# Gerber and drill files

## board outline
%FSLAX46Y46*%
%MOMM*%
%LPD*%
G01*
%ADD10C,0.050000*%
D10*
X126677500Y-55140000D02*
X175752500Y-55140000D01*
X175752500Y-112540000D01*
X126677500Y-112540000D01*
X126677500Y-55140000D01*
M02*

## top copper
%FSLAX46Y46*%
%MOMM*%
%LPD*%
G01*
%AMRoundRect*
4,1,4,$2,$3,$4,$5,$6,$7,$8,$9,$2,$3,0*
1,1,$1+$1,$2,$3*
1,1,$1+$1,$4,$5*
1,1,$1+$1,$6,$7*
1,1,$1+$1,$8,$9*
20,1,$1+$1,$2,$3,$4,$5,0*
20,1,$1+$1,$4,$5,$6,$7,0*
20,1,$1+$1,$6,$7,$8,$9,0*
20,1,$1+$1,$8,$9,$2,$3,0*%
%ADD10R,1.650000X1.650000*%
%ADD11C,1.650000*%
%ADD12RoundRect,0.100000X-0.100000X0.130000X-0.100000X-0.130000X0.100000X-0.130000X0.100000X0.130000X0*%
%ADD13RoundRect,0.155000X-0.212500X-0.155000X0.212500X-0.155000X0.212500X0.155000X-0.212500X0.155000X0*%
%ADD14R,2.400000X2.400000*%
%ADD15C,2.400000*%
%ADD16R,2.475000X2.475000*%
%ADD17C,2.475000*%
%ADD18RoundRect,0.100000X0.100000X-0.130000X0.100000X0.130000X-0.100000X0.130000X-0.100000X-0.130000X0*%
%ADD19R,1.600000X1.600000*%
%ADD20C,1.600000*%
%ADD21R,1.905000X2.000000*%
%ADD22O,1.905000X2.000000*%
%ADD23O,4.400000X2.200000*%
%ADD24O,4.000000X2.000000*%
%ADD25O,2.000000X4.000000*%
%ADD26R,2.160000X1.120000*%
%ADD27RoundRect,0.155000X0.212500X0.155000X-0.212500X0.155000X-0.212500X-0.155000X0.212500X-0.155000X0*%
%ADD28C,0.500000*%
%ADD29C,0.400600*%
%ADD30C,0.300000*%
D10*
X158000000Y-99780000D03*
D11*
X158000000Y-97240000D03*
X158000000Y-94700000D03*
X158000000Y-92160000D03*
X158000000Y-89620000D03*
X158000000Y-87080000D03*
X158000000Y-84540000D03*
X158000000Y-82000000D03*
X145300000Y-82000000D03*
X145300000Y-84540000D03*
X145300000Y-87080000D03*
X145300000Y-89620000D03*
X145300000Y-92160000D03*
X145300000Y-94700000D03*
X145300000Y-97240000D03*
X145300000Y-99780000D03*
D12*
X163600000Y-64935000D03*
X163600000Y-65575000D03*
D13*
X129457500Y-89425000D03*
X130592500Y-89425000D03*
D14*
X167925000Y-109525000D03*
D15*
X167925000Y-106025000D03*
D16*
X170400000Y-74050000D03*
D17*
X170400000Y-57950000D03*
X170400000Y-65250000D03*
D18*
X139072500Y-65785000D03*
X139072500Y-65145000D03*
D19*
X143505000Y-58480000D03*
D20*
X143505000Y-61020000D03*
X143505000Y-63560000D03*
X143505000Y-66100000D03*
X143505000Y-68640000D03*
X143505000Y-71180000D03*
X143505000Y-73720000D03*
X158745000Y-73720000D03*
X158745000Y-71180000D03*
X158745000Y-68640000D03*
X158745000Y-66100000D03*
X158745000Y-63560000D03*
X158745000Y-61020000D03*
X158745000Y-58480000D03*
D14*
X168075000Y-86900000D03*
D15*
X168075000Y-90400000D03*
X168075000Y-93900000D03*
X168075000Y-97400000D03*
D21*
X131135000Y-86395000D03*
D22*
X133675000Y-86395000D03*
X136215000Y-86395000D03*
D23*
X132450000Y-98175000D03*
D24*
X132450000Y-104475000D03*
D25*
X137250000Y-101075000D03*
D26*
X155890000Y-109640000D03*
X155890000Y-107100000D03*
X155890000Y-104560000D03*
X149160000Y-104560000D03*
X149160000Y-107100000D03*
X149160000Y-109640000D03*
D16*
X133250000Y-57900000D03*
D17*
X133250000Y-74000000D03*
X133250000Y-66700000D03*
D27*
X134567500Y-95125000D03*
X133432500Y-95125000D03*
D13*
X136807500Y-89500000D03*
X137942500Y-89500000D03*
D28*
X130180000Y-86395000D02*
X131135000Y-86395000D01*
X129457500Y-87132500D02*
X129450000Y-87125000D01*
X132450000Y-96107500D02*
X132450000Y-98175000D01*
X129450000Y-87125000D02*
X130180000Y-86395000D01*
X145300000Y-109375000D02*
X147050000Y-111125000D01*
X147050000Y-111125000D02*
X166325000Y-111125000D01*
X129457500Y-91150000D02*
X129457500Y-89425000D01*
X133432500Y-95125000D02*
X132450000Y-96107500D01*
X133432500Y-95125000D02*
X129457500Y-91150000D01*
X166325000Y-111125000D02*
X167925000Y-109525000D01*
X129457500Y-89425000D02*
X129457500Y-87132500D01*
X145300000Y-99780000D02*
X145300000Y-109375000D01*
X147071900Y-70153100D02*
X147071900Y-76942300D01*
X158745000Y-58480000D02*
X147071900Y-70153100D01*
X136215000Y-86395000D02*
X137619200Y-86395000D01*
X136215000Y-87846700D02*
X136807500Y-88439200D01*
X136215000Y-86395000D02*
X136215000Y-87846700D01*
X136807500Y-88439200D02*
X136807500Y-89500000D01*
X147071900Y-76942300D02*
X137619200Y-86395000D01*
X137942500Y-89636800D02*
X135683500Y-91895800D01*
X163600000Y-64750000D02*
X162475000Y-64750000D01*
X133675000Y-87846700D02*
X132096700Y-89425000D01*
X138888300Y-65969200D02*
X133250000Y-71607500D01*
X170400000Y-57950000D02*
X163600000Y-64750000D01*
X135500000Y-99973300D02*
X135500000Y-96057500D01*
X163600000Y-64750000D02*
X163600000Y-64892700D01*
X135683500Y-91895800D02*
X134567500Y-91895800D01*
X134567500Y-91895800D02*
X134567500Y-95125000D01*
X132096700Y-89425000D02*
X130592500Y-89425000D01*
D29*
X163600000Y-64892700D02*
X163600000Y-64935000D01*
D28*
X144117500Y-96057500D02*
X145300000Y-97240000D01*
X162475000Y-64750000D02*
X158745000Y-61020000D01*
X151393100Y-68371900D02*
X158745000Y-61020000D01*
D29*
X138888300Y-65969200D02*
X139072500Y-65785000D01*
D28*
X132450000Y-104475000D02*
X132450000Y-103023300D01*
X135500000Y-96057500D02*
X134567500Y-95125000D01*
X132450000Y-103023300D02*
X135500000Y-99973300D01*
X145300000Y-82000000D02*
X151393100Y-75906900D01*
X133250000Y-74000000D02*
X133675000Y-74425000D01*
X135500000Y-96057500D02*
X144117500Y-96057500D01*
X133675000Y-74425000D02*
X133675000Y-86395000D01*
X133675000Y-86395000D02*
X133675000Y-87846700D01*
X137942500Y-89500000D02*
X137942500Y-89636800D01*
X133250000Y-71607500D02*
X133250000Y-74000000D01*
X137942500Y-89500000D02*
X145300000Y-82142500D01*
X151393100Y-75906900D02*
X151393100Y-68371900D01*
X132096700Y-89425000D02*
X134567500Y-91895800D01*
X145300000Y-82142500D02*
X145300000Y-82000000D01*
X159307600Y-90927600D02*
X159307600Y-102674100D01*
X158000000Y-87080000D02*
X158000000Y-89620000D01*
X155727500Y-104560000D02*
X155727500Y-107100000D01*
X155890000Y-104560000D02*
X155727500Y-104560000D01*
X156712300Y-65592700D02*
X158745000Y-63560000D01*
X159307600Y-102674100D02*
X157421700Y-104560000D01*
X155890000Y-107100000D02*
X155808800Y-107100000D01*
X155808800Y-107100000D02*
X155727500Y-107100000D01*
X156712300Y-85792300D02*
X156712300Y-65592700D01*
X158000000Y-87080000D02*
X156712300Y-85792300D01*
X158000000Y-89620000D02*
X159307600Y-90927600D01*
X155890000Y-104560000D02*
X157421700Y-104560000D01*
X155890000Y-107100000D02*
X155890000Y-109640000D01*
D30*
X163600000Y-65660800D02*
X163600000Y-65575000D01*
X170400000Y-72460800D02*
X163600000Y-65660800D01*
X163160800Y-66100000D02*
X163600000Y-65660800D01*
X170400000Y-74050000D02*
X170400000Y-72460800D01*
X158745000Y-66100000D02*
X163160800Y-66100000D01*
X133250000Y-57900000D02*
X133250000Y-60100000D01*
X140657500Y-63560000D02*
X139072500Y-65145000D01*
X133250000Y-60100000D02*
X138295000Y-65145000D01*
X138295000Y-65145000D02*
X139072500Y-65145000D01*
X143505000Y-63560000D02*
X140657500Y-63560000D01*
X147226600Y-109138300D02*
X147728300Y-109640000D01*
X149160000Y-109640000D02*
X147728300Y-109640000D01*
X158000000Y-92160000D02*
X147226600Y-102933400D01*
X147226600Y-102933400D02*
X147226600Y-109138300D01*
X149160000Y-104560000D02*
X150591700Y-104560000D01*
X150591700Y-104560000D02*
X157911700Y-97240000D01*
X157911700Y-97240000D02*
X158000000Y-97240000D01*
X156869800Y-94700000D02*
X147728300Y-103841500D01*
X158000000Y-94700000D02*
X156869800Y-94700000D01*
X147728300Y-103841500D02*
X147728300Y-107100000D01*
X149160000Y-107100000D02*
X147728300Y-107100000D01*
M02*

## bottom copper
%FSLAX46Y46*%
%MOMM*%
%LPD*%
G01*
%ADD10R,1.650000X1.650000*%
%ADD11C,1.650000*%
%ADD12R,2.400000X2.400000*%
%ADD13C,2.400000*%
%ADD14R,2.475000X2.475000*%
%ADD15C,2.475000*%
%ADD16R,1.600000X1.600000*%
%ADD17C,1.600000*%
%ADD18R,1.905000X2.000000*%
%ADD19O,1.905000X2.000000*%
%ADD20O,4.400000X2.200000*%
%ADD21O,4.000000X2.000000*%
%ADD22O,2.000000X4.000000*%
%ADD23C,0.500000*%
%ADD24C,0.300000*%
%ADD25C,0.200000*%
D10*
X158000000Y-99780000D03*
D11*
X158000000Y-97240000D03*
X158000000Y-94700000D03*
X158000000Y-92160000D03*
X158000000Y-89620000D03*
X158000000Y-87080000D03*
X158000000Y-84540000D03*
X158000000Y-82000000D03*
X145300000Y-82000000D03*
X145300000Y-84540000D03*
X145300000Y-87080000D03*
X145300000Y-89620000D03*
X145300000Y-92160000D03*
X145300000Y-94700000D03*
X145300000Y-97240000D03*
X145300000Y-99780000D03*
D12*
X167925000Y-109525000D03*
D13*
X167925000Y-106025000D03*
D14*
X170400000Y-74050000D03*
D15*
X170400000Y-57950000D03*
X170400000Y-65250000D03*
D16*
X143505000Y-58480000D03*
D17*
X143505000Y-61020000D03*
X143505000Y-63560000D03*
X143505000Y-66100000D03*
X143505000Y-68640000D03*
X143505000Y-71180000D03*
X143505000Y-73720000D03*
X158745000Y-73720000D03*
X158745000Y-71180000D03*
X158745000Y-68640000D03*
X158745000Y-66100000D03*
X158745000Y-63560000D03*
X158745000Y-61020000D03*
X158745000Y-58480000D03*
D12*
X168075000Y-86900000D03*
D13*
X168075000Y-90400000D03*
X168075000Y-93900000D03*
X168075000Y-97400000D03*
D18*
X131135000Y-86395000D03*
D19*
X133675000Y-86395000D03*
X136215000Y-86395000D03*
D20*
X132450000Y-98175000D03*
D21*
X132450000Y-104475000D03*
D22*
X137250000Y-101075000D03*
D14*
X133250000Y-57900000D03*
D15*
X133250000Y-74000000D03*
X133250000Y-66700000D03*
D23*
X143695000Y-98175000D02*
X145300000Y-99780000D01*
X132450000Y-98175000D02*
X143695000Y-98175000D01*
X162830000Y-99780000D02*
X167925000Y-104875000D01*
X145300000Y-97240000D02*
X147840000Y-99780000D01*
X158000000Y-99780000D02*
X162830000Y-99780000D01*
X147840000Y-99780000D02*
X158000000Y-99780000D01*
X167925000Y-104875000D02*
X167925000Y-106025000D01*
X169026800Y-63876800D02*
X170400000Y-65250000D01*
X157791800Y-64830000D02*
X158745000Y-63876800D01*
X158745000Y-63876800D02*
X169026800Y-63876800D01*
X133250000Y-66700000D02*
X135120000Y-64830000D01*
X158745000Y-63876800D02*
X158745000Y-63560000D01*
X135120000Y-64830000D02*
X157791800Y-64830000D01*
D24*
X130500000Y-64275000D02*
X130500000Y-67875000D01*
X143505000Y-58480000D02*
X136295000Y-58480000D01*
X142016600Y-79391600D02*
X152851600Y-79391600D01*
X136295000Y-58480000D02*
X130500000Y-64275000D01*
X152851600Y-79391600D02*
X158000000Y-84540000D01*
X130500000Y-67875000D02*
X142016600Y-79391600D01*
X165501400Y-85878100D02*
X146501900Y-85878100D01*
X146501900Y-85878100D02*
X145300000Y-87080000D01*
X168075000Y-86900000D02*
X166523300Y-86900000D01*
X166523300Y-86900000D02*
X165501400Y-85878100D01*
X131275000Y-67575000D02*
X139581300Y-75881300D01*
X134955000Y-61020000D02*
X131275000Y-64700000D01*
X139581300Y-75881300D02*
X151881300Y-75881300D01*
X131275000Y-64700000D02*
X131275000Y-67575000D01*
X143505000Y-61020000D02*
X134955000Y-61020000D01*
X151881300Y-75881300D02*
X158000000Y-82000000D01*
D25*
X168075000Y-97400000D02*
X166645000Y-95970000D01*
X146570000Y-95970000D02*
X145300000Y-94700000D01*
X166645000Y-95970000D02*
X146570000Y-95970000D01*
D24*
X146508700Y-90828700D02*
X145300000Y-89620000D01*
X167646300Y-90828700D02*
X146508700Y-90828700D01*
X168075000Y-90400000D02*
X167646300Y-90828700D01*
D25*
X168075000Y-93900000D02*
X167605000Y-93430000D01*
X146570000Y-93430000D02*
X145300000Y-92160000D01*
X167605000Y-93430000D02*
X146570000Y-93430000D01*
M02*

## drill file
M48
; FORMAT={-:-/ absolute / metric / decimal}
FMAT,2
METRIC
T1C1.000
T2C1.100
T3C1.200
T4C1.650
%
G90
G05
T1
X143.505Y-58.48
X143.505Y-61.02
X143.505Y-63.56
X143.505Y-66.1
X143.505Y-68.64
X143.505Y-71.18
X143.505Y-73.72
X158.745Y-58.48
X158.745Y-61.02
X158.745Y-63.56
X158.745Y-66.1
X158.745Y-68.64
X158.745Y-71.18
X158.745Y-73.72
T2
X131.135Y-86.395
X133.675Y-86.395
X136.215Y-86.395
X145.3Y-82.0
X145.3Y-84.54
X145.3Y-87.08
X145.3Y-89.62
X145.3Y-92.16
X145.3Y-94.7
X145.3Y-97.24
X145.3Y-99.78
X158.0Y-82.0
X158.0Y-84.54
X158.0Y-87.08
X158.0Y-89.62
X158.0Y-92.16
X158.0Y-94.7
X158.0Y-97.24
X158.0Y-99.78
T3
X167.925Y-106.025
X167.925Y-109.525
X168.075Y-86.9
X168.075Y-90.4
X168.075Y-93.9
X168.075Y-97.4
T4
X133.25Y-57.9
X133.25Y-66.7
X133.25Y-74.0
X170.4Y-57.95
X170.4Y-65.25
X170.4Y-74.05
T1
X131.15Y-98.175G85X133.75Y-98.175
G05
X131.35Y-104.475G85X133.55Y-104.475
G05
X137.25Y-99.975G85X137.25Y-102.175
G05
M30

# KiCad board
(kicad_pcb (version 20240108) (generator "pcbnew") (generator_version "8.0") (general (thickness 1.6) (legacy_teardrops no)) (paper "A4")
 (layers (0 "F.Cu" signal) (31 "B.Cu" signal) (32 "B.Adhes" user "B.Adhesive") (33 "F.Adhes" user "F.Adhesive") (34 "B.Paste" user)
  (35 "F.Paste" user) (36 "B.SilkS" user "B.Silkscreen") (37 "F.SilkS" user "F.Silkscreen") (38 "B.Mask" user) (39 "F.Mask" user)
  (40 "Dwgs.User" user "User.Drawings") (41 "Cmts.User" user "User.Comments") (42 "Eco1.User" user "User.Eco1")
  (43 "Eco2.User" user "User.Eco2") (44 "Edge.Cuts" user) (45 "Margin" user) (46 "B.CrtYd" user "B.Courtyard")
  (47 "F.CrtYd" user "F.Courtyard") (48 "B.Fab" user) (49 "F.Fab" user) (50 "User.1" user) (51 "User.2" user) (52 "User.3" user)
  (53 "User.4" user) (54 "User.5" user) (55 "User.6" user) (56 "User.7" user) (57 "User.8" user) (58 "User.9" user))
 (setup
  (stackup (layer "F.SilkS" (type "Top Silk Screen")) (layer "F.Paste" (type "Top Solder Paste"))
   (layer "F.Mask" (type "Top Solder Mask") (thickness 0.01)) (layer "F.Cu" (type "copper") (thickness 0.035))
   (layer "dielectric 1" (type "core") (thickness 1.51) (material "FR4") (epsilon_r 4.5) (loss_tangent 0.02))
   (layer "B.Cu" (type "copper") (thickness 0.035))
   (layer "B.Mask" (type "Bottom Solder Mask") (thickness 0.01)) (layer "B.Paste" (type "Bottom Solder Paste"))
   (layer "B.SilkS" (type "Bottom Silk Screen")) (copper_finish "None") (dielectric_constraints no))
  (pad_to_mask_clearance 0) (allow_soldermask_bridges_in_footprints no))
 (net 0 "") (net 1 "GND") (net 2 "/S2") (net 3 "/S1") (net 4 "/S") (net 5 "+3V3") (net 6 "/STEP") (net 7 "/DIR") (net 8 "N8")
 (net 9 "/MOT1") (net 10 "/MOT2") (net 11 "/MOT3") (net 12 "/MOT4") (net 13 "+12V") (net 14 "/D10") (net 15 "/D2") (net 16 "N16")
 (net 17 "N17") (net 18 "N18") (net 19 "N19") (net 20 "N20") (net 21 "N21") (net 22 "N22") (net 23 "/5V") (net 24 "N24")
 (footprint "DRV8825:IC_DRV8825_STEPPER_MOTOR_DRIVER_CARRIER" (layer "F.Cu") (at 151.65 90.89 180)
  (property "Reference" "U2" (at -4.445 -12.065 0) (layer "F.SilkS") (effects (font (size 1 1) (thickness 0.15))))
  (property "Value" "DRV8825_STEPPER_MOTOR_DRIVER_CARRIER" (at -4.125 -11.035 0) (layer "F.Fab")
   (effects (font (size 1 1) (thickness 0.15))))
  (pad "1" thru_hole rect (at -6.35 -8.89 180) (size 1.65 1.65) (drill 1.1) (layers "*.Cu" "*.Mask") (remove_unused_layers no) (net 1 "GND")
   (solder_mask_margin 0.102))
  (pad "2" thru_hole circle (at -6.35 -6.35 180) (size 1.65 1.65) (drill 1.1) (layers "*.Cu" "*.Mask") (remove_unused_layers no)
   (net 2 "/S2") (solder_mask_margin 0.102))
  (pad "3" thru_hole circle (at -6.35 -3.81 180) (size 1.65 1.65) (drill 1.1) (layers "*.Cu" "*.Mask") (remove_unused_layers no)
   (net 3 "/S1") (solder_mask_margin 0.102))
  (pad "4" thru_hole circle (at -6.35 -1.27 180) (size 1.65 1.65) (drill 1.1) (layers "*.Cu" "*.Mask") (remove_unused_layers no)
   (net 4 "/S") (solder_mask_margin 0.102))
  (pad "5" thru_hole circle (at -6.35 1.27 180) (size 1.65 1.65) (drill 1.1) (layers "*.Cu" "*.Mask") (remove_unused_layers no)
   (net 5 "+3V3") (solder_mask_margin 0.102))
  (pad "6" thru_hole circle (at -6.35 3.81 180) (size 1.65 1.65) (drill 1.1) (layers "*.Cu" "*.Mask") (remove_unused_layers no)
   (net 5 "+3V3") (solder_mask_margin 0.102))
  (pad "7" thru_hole circle (at -6.35 6.35 180) (size 1.65 1.65) (drill 1.1) (layers "*.Cu" "*.Mask") (remove_unused_layers no)
   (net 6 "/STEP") (solder_mask_margin 0.102))
  (pad "8" thru_hole circle (at -6.35 8.89 180) (size 1.65 1.65) (drill 1.1) (layers "*.Cu" "*.Mask") (remove_unused_layers no)
   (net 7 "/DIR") (solder_mask_margin 0.102))
  (pad "9" thru_hole circle (at 6.35 8.89 180) (size 1.65 1.65) (drill 1.1) (layers "*.Cu" "*.Mask") (remove_unused_layers no) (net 1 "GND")
   (solder_mask_margin 0.102))
  (pad "10" thru_hole circle (at 6.35 6.35 180) (size 1.65 1.65) (drill 1.1) (layers "*.Cu" "*.Mask") (remove_unused_layers no) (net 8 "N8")
   (solder_mask_margin 0.102))
  (pad "11" thru_hole circle (at 6.35 3.81 180) (size 1.65 1.65) (drill 1.1) (layers "*.Cu" "*.Mask") (remove_unused_layers no)
   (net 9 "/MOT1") (solder_mask_margin 0.102))
  (pad "12" thru_hole circle (at 6.35 1.27 180) (size 1.65 1.65) (drill 1.1) (layers "*.Cu" "*.Mask") (remove_unused_layers no)
   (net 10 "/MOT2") (solder_mask_margin 0.102))
  (pad "13" thru_hole circle (at 6.35 -1.27 180) (size 1.65 1.65) (drill 1.1) (layers "*.Cu" "*.Mask") (remove_unused_layers no)
   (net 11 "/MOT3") (solder_mask_margin 0.102))
  (pad "14" thru_hole circle (at 6.35 -3.81 180) (size 1.65 1.65) (drill 1.1) (layers "*.Cu" "*.Mask") (remove_unused_layers no)
   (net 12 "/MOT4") (solder_mask_margin 0.102))
  (pad "15" thru_hole circle (at 6.35 -6.35 180) (size 1.65 1.65) (drill 1.1) (layers "*.Cu" "*.Mask") (remove_unused_layers no)
   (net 1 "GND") (solder_mask_margin 0.102))
  (pad "16" thru_hole circle (at 6.35 -8.89 180) (size 1.65 1.65) (drill 1.1) (layers "*.Cu" "*.Mask") (remove_unused_layers no)
   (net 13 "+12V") (solder_mask_margin 0.102)))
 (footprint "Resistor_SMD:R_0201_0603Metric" (layer "F.Cu") (at 163.6 65.255 -90)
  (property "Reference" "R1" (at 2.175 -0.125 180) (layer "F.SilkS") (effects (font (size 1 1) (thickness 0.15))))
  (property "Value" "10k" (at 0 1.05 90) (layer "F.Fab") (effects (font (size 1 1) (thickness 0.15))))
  (pad "" smd roundrect (at -0.345 0 270) (size 0.318 0.36) (layers "F.Paste") (roundrect_rratio 0.25))
  (pad "" smd roundrect (at 0.345 0 270) (size 0.318 0.36) (layers "F.Paste") (roundrect_rratio 0.25))
  (pad "1" smd roundrect (at -0.32 0 270) (size 0.46 0.4) (layers "F.Cu" "F.Mask") (roundrect_rratio 0.25) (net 1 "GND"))
  (pad "2" smd roundrect (at 0.32 0 270) (size 0.46 0.4) (layers "F.Cu" "F.Mask") (roundrect_rratio 0.25) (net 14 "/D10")))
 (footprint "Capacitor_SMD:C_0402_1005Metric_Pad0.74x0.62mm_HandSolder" (layer "F.Cu") (at 130.025 89.425)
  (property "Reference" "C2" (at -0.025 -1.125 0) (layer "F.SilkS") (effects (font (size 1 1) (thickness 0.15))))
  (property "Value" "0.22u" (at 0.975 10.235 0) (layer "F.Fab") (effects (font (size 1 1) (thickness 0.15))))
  (pad "1" smd roundrect (at -0.5675 0) (size 0.735 0.62) (layers "F.Cu" "F.Paste" "F.Mask") (roundrect_rratio 0.25) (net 13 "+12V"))
  (pad "2" smd roundrect (at 0.5675 0) (size 0.735 0.62) (layers "F.Cu" "F.Paste" "F.Mask") (roundrect_rratio 0.25) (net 1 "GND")))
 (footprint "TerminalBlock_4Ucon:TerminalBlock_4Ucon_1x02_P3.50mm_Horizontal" (layer "F.Cu") (at 167.925 109.525 90)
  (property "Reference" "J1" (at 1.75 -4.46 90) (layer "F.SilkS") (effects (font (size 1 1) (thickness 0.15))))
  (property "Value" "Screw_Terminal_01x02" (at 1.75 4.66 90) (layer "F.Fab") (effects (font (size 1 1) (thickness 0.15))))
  (pad "1" thru_hole rect (at 0 0 90) (size 2.4 2.4) (drill 1.2) (layers "*.Cu" "*.Mask") (remove_unused_layers no) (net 13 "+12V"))
  (pad "2" thru_hole circle (at 3.5 0 90) (size 2.4 2.4) (drill 1.2) (layers "*.Cu" "*.Mask") (remove_unused_layers no) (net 1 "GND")))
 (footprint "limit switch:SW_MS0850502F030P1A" (layer "F.Cu") (at 170.4 74.05 90)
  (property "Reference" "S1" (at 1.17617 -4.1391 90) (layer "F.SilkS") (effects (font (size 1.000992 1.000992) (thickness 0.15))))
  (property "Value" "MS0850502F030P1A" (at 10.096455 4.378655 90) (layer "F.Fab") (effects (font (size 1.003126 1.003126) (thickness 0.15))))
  (pad "1" thru_hole rect (at 0 0 90) (size 2.475 2.475) (drill 1.65) (layers "*.Cu" "*.Mask") (remove_unused_layers no) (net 14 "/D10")
   (solder_mask_margin 0.102))
  (pad "2" thru_hole circle (at 16.1 0 90) (size 2.475 2.475) (drill 1.65) (layers "*.Cu" "*.Mask") (remove_unused_layers no) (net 1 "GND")
   (solder_mask_margin 0.102))
  (pad "3" thru_hole circle (at 8.8 0 90) (size 2.475 2.475) (drill 1.65) (layers "*.Cu" "*.Mask") (remove_unused_layers no) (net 5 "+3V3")
   (solder_mask_margin 0.102)))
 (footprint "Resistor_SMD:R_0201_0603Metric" (layer "F.Cu") (at 139.0725 65.465 90)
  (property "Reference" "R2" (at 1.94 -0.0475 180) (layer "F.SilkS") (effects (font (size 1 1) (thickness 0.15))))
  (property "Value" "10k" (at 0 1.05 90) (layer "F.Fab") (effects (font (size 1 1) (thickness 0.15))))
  (pad "" smd roundrect (at -0.345 0 90) (size 0.318 0.36) (layers "F.Paste") (roundrect_rratio 0.25))
  (pad "" smd roundrect (at 0.345 0 90) (size 0.318 0.36) (layers "F.Paste") (roundrect_rratio 0.25))
  (pad "1" smd roundrect (at -0.32 0 90) (size 0.46 0.4) (layers "F.Cu" "F.Mask") (roundrect_rratio 0.25) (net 1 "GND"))
  (pad "2" smd roundrect (at 0.32 0 90) (size 0.46 0.4) (layers "F.Cu" "F.Mask") (roundrect_rratio 0.25) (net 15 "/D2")))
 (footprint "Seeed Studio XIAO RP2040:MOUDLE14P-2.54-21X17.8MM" (layer "F.Cu") (at 151.125 66.1 90)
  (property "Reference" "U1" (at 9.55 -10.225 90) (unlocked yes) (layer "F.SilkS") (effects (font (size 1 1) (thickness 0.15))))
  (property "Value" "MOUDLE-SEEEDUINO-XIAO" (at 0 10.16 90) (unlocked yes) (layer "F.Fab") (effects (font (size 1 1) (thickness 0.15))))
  (pad "1" thru_hole rect (at 7.62 -7.62 90) (size 1.6 1.6) (drill 1) (layers "*.Cu" "*.Mask") (remove_unused_layers no) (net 6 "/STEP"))
  (pad "2" thru_hole circle (at 5.08 -7.62 90) (size 1.6 1.6) (drill 1) (layers "*.Cu" "*.Mask") (remove_unused_layers no) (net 7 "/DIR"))
  (pad "3" thru_hole circle (at 2.54 -7.62 90) (size 1.6 1.6) (drill 1) (layers "*.Cu" "*.Mask") (remove_unused_layers no) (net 15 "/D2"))
  (pad "4" thru_hole circle (at 0 -7.62 90) (size 1.6 1.6) (drill 1) (layers "*.Cu" "*.Mask") (remove_unused_layers no) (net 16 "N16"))
  (pad "5" thru_hole circle (at -2.54 -7.62 90) (size 1.6 1.6) (drill 1) (layers "*.Cu" "*.Mask") (remove_unused_layers no) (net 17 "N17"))
  (pad "6" thru_hole circle (at -5.08 -7.62 90) (size 1.6 1.6) (drill 1) (layers "*.Cu" "*.Mask") (remove_unused_layers no) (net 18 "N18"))
  (pad "7" thru_hole circle (at -7.62 -7.62 90) (size 1.6 1.6) (drill 1) (layers "*.Cu" "*.Mask") (remove_unused_layers no) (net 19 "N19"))
  (pad "8" thru_hole circle (at -7.62 7.62 90) (size 1.6 1.6) (drill 1) (layers "*.Cu" "*.Mask") (remove_unused_layers no) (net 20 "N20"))
  (pad "9" thru_hole circle (at -5.08 7.62 90) (size 1.6 1.6) (drill 1) (layers "*.Cu" "*.Mask") (remove_unused_layers no) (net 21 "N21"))
  (pad "10" thru_hole circle (at -2.54 7.62 90) (size 1.6 1.6) (drill 1) (layers "*.Cu" "*.Mask") (remove_unused_layers no) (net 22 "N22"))
  (pad "11" thru_hole circle (at 0 7.62 90) (size 1.6 1.6) (drill 1) (layers "*.Cu" "*.Mask") (remove_unused_layers no) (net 14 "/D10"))
  (pad "12" thru_hole circle (at 2.54 7.62 90) (size 1.6 1.6) (drill 1) (layers "*.Cu" "*.Mask") (remove_unused_layers no) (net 5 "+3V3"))
  (pad "13" thru_hole circle (at 5.08 7.62 90) (size 1.6 1.6) (drill 1) (layers "*.Cu" "*.Mask") (remove_unused_layers no) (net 1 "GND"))
  (pad "14" thru_hole circle (at 7.62 7.62 90) (size 1.6 1.6) (drill 1) (layers "*.Cu" "*.Mask") (remove_unused_layers no) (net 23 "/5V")))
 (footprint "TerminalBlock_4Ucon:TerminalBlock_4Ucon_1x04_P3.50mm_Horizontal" (layer "F.Cu") (at 168.075 86.9 -90)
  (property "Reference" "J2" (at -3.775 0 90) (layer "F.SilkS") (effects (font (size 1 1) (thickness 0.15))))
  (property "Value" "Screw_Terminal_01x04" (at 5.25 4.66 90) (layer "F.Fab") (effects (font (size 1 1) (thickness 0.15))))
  (pad "1" thru_hole rect (at 0 0 270) (size 2.4 2.4) (drill 1.2) (layers "*.Cu" "*.Mask") (remove_unused_layers no) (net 9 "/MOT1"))
  (pad "2" thru_hole circle (at 3.5 0 270) (size 2.4 2.4) (drill 1.2) (layers "*.Cu" "*.Mask") (remove_unused_layers no) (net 10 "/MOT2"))
  (pad "3" thru_hole circle (at 7 0 270) (size 2.4 2.4) (drill 1.2) (layers "*.Cu" "*.Mask") (remove_unused_layers no) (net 11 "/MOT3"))
  (pad "4" thru_hole circle (at 10.5 0 270) (size 2.4 2.4) (drill 1.2) (layers "*.Cu" "*.Mask") (remove_unused_layers no) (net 12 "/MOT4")))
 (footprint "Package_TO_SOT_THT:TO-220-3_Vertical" (layer "F.Cu") (at 131.135 86.395)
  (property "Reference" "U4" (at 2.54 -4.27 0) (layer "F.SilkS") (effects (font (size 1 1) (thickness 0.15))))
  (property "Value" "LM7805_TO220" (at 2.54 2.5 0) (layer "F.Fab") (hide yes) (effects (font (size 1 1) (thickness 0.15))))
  (pad "1" thru_hole rect (at 0 0) (size 1.905 2) (drill 1.1) (layers "*.Cu" "*.Mask") (remove_unused_layers no) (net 13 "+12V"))
  (pad "2" thru_hole oval (at 2.54 0) (size 1.905 2) (drill 1.1) (layers "*.Cu" "*.Mask") (remove_unused_layers no) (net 1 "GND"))
  (pad "3" thru_hole oval (at 5.08 0) (size 1.905 2) (drill 1.1) (layers "*.Cu" "*.Mask") (remove_unused_layers no) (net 23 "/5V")))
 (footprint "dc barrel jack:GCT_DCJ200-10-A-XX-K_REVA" (layer "F.Cu") (at 132.45 104.725)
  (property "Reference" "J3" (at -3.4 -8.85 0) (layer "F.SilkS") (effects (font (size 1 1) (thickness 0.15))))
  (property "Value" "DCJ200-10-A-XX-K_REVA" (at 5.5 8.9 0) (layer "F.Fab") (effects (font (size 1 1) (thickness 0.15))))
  (pad "1" thru_hole oval (at 0 -6.55) (size 4.4 2.2) (drill oval 3.6 1) (layers "*.Cu" "*.Mask") (remove_unused_layers no) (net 13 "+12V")
   (solder_mask_margin 0.102))
  (pad "2" thru_hole oval (at 0 -0.25) (size 4 2) (drill oval 3.2 1) (layers "*.Cu" "*.Mask") (remove_unused_layers no) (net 1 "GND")
   (solder_mask_margin 0.102))
  (pad "3" thru_hole oval (at 4.8 -3.65) (size 2 4) (drill oval 1 3.2) (layers "*.Cu" "*.Mask") (remove_unused_layers no) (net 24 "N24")
   (solder_mask_margin 0.102)))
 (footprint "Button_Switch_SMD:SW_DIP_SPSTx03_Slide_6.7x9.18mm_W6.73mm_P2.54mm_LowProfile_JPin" (layer "F.Cu") (at 152.525 107.1 180)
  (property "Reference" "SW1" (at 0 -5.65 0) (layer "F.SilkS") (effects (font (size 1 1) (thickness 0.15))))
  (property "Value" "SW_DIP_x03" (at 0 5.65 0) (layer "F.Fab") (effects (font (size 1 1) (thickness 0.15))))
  (pad "1" smd rect (at -3.365 -2.54 180) (size 2.16 1.12) (layers "F.Cu" "F.Paste" "F.Mask") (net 5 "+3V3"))
  (pad "2" smd rect (at -3.365 0 180) (size 2.16 1.12) (layers "F.Cu" "F.Paste" "F.Mask") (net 5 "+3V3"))
  (pad "3" smd rect (at -3.365 2.54 180) (size 2.16 1.12) (layers "F.Cu" "F.Paste" "F.Mask") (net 5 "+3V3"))
  (pad "4" smd rect (at 3.365 2.54 180) (size 2.16 1.12) (layers "F.Cu" "F.Paste" "F.Mask") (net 2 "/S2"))
  (pad "5" smd rect (at 3.365 0 180) (size 2.16 1.12) (layers "F.Cu" "F.Paste" "F.Mask") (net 3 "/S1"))
  (pad "6" smd rect (at 3.365 -2.54 180) (size 2.16 1.12) (layers "F.Cu" "F.Paste" "F.Mask") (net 4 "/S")))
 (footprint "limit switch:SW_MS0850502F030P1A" (layer "F.Cu") (at 133.25 57.9 -90)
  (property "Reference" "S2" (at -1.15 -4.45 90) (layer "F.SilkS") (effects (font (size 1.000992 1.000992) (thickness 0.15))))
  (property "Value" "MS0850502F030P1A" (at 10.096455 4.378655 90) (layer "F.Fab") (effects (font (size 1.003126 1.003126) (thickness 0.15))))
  (pad "1" thru_hole rect (at 0 0 270) (size 2.475 2.475) (drill 1.65) (layers "*.Cu" "*.Mask") (remove_unused_layers no) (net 15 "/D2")
   (solder_mask_margin 0.102))
  (pad "2" thru_hole circle (at 16.1 0 270) (size 2.475 2.475) (drill 1.65) (layers "*.Cu" "*.Mask") (remove_unused_layers no) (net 1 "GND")
   (solder_mask_margin 0.102))
  (pad "3" thru_hole circle (at 8.8 0 270) (size 2.475 2.475) (drill 1.65) (layers "*.Cu" "*.Mask") (remove_unused_layers no) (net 5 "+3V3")
   (solder_mask_margin 0.102)))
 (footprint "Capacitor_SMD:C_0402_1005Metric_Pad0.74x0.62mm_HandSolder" (layer "F.Cu") (at 134 95.125 180)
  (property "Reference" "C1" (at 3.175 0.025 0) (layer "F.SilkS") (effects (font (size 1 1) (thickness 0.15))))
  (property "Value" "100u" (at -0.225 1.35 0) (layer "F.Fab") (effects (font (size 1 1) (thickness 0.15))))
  (pad "1" smd roundrect (at -0.5675 0 180) (size 0.735 0.62) (layers "F.Cu" "F.Paste" "F.Mask") (roundrect_rratio 0.25) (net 1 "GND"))
  (pad "2" smd roundrect (at 0.5675 0 180) (size 0.735 0.62) (layers "F.Cu" "F.Paste" "F.Mask") (roundrect_rratio 0.25) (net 13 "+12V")))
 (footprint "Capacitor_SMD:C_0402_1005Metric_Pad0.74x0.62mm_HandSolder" (layer "F.Cu") (at 137.375 89.5)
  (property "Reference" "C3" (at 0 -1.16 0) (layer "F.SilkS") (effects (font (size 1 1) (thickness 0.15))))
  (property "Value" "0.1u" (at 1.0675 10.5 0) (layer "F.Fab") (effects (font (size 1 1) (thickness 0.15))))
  (pad "1" smd roundrect (at -0.5675 0) (size 0.735 0.62) (layers "F.Cu" "F.Paste" "F.Mask") (roundrect_rratio 0.25) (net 23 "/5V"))
  (pad "2" smd roundrect (at 0.5675 0) (size 0.735 0.62) (layers "F.Cu" "F.Paste" "F.Mask") (roundrect_rratio 0.25) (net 1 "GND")))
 (gr_rect (start 126.6775 55.14) (end 175.7525 112.54) (stroke (width 0.05) (type default)) (fill none) (layer "Edge.Cuts"))
 (segment (start 130.18 86.395) (end 131.135 86.395) (width 0.5) (layer "F.Cu") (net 13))
 (segment (start 129.4575 87.1325) (end 129.45 87.125) (width 0.5) (layer "F.Cu") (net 13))
 (segment (start 132.45 96.1075) (end 132.45 98.175) (width 0.5) (layer "F.Cu") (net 13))
 (segment (start 129.45 87.125) (end 130.18 86.395) (width 0.5) (layer "F.Cu") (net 13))
 (segment (start 145.3 109.375) (end 147.05 111.125) (width 0.5) (layer "F.Cu") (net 13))
 (segment (start 147.05 111.125) (end 166.325 111.125) (width 0.5) (layer "F.Cu") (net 13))
 (segment (start 129.4575 91.15) (end 129.4575 89.425) (width 0.5) (layer "F.Cu") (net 13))
 (segment (start 133.4325 95.125) (end 132.45 96.1075) (width 0.5) (layer "F.Cu") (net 13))
 (segment (start 133.4325 95.125) (end 129.4575 91.15) (width 0.5) (layer "F.Cu") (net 13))
 (segment (start 166.325 111.125) (end 167.925 109.525) (width 0.5) (layer "F.Cu") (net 13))
 (segment (start 129.4575 89.425) (end 129.4575 87.1325) (width 0.5) (layer "F.Cu") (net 13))
 (segment (start 145.3 99.78) (end 145.3 109.375) (width 0.5) (layer "F.Cu") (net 13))
 (segment (start 143.695 98.175) (end 145.3 99.78) (width 0.5) (layer "B.Cu") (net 13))
 (segment (start 132.45 98.175) (end 143.695 98.175) (width 0.5) (layer "B.Cu") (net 13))
 (segment (start 147.0719 70.1531) (end 147.0719 76.9423) (width 0.5) (layer "F.Cu") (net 23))
 (segment (start 158.745 58.48) (end 147.0719 70.1531) (width 0.5) (layer "F.Cu") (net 23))
 (segment (start 136.215 86.395) (end 137.6192 86.395) (width 0.5) (layer "F.Cu") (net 23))
 (segment (start 136.215 87.8467) (end 136.8075 88.4392) (width 0.5) (layer "F.Cu") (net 23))
 (segment (start 136.215 86.395) (end 136.215 87.8467) (width 0.5) (layer "F.Cu") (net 23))
 (segment (start 136.8075 88.4392) (end 136.8075 89.5) (width 0.5) (layer "F.Cu") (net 23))
 (segment (start 147.0719 76.9423) (end 137.6192 86.395) (width 0.5) (layer "F.Cu") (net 23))
 (segment (start 137.9425 89.6368) (end 135.6835 91.8958) (width 0.5) (layer "F.Cu") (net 1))
 (segment (start 163.6 64.75) (end 162.475 64.75) (width 0.5) (layer "F.Cu") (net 1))
 (segment (start 133.675 87.8467) (end 132.0967 89.425) (width 0.5) (layer "F.Cu") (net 1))
 (segment (start 138.8883 65.9692) (end 133.25 71.6075) (width 0.5) (layer "F.Cu") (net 1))
 (segment (start 170.4 57.95) (end 163.6 64.75) (width 0.5) (layer "F.Cu") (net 1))
 (segment (start 135.5 99.9733) (end 135.5 96.0575) (width 0.5) (layer "F.Cu") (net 1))
 (segment (start 163.6 64.75) (end 163.6 64.8927) (width 0.5) (layer "F.Cu") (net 1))
 (segment (start 135.6835 91.8958) (end 134.5675 91.8958) (width 0.5) (layer "F.Cu") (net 1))
 (segment (start 134.5675 91.8958) (end 134.5675 95.125) (width 0.5) (layer "F.Cu") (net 1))
 (segment (start 132.0967 89.425) (end 130.5925 89.425) (width 0.5) (layer "F.Cu") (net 1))
 (segment (start 163.6 64.8927) (end 163.6 64.935) (width 0.4006) (layer "F.Cu") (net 1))
 (segment (start 144.1175 96.0575) (end 145.3 97.24) (width 0.5) (layer "F.Cu") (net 1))
 (segment (start 162.475 64.75) (end 158.745 61.02) (width 0.5) (layer "F.Cu") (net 1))
 (segment (start 151.3931 68.3719) (end 158.745 61.02) (width 0.5) (layer "F.Cu") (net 1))
 (segment (start 138.8883 65.9692) (end 139.0725 65.785) (width 0.4006) (layer "F.Cu") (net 1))
 (segment (start 132.45 104.475) (end 132.45 103.0233) (width 0.5) (layer "F.Cu") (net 1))
 (segment (start 135.5 96.0575) (end 134.5675 95.125) (width 0.5) (layer "F.Cu") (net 1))
 (segment (start 132.45 103.0233) (end 135.5 99.9733) (width 0.5) (layer "F.Cu") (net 1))
 (segment (start 145.3 82) (end 151.3931 75.9069) (width 0.5) (layer "F.Cu") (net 1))
 (segment (start 133.25 74) (end 133.675 74.425) (width 0.5) (layer "F.Cu") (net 1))
 (segment (start 135.5 96.0575) (end 144.1175 96.0575) (width 0.5) (layer "F.Cu") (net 1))
 (segment (start 133.675 74.425) (end 133.675 86.395) (width 0.5) (layer "F.Cu") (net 1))
 (segment (start 133.675 86.395) (end 133.675 87.8467) (width 0.5) (layer "F.Cu") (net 1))
 (segment (start 137.9425 89.5) (end 137.9425 89.6368) (width 0.5) (layer "F.Cu") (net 1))
 (segment (start 133.25 71.6075) (end 133.25 74) (width 0.5) (layer "F.Cu") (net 1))
 (segment (start 137.9425 89.5) (end 145.3 82.1425) (width 0.5) (layer "F.Cu") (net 1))
 (segment (start 151.3931 75.9069) (end 151.3931 68.3719) (width 0.5) (layer "F.Cu") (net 1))
 (segment (start 132.0967 89.425) (end 134.5675 91.8958) (width 0.5) (layer "F.Cu") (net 1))
 (segment (start 145.3 82.1425) (end 145.3 82) (width 0.5) (layer "F.Cu") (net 1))
 (segment (start 162.83 99.78) (end 167.925 104.875) (width 0.5) (layer "B.Cu") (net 1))
 (segment (start 145.3 97.24) (end 147.84 99.78) (width 0.5) (layer "B.Cu") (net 1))
 (segment (start 158 99.78) (end 162.83 99.78) (width 0.5) (layer "B.Cu") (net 1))
 (segment (start 147.84 99.78) (end 158 99.78) (width 0.5) (layer "B.Cu") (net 1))
 (segment (start 167.925 104.875) (end 167.925 106.025) (width 0.5) (layer "B.Cu") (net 1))
 (segment (start 159.3076 90.9276) (end 159.3076 102.6741) (width 0.5) (layer "F.Cu") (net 5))
 (segment (start 158 87.08) (end 158 89.62) (width 0.5) (layer "F.Cu") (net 5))
 (segment (start 155.7275 104.56) (end 155.7275 107.1) (width 0.5) (layer "F.Cu") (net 5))
 (segment (start 155.89 104.56) (end 155.7275 104.56) (width 0.5) (layer "F.Cu") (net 5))
 (segment (start 156.7123 65.5927) (end 158.745 63.56) (width 0.5) (layer "F.Cu") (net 5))
 (segment (start 159.3076 102.6741) (end 157.4217 104.56) (width 0.5) (layer "F.Cu") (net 5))
 (segment (start 155.89 107.1) (end 155.8088 107.1) (width 0.5) (layer "F.Cu") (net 5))
 (segment (start 155.8088 107.1) (end 155.7275 107.1) (width 0.5) (layer "F.Cu") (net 5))
 (segment (start 156.7123 85.7923) (end 156.7123 65.5927) (width 0.5) (layer "F.Cu") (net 5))
 (segment (start 158 87.08) (end 156.7123 85.7923) (width 0.5) (layer "F.Cu") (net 5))
 (segment (start 158 89.62) (end 159.3076 90.9276) (width 0.5) (layer "F.Cu") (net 5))
 (segment (start 155.89 104.56) (end 157.4217 104.56) (width 0.5) (layer "F.Cu") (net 5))
 (segment (start 155.89 107.1) (end 155.89 109.64) (width 0.5) (layer "F.Cu") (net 5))
 (segment (start 169.0268 63.8768) (end 170.4 65.25) (width 0.5) (layer "B.Cu") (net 5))
 (segment (start 157.7918 64.83) (end 158.745 63.8768) (width 0.5) (layer "B.Cu") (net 5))
 (segment (start 158.745 63.8768) (end 169.0268 63.8768) (width 0.5) (layer "B.Cu") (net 5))
 (segment (start 133.25 66.7) (end 135.12 64.83) (width 0.5) (layer "B.Cu") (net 5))
 (segment (start 158.745 63.8768) (end 158.745 63.56) (width 0.5) (layer "B.Cu") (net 5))
 (segment (start 135.12 64.83) (end 157.7918 64.83) (width 0.5) (layer "B.Cu") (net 5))
 (segment (start 163.6 65.6608) (end 163.6 65.575) (width 0.3) (layer "F.Cu") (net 14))
 (segment (start 170.4 72.4608) (end 163.6 65.6608) (width 0.3) (layer "F.Cu") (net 14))
 (segment (start 163.1608 66.1) (end 163.6 65.6608) (width 0.3) (layer "F.Cu") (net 14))
 (segment (start 170.4 74.05) (end 170.4 72.4608) (width 0.3) (layer "F.Cu") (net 14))
 (segment (start 158.745 66.1) (end 163.1608 66.1) (width 0.3) (layer "F.Cu") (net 14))
 (segment (start 130.5 64.275) (end 130.5 67.875) (width 0.3) (layer "B.Cu") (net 6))
 (segment (start 143.505 58.48) (end 136.295 58.48) (width 0.3) (layer "B.Cu") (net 6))
 (segment (start 142.0166 79.3916) (end 152.8516 79.3916) (width 0.3) (layer "B.Cu") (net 6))
 (segment (start 136.295 58.48) (end 130.5 64.275) (width 0.3) (layer "B.Cu") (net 6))
 (segment (start 152.8516 79.3916) (end 158 84.54) (width 0.3) (layer "B.Cu") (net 6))
 (segment (start 130.5 67.875) (end 142.0166 79.3916) (width 0.3) (layer "B.Cu") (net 6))
 (segment (start 133.25 57.9) (end 133.25 60.1) (width 0.3) (layer "F.Cu") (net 15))
 (segment (start 140.6575 63.56) (end 139.0725 65.145) (width 0.3) (layer "F.Cu") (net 15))
 (segment (start 133.25 60.1) (end 138.295 65.145) (width 0.3) (layer "F.Cu") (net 15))
 (segment (start 138.295 65.145) (end 139.0725 65.145) (width 0.3) (layer "F.Cu") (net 15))
 (segment (start 143.505 63.56) (end 140.6575 63.56) (width 0.3) (layer "F.Cu") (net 15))
 (segment (start 165.5014 85.8781) (end 146.5019 85.8781) (width 0.3) (layer "B.Cu") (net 9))
 (segment (start 146.5019 85.8781) (end 145.3 87.08) (width 0.3) (layer "B.Cu") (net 9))
 (segment (start 168.075 86.9) (end 166.5233 86.9) (width 0.3) (layer "B.Cu") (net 9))
 (segment (start 166.5233 86.9) (end 165.5014 85.8781) (width 0.3) (layer "B.Cu") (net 9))
 (segment (start 147.2266 109.1383) (end 147.7283 109.64) (width 0.3) (layer "F.Cu") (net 4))
 (segment (start 149.16 109.64) (end 147.7283 109.64) (width 0.3) (layer "F.Cu") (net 4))
 (segment (start 158 92.16) (end 147.2266 102.9334) (width 0.3) (layer "F.Cu") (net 4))
 (segment (start 147.2266 102.9334) (end 147.2266 109.1383) (width 0.3) (layer "F.Cu") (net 4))
 (segment (start 131.275 67.575) (end 139.5813 75.8813) (width 0.3) (layer "B.Cu") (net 7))
 (segment (start 134.955 61.02) (end 131.275 64.7) (width 0.3) (layer "B.Cu") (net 7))
 (segment (start 139.5813 75.8813) (end 151.8813 75.8813) (width 0.3) (layer "B.Cu") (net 7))
 (segment (start 131.275 64.7) (end 131.275 67.575) (width 0.3) (layer "B.Cu") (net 7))
 (segment (start 143.505 61.02) (end 134.955 61.02) (width 0.3) (layer "B.Cu") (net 7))
 (segment (start 151.8813 75.8813) (end 158 82) (width 0.3) (layer "B.Cu") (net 7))
 (segment (start 168.075 97.4) (end 166.645 95.97) (width 0.2) (layer "B.Cu") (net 12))
 (segment (start 146.57 95.97) (end 145.3 94.7) (width 0.2) (layer "B.Cu") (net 12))
 (segment (start 166.645 95.97) (end 146.57 95.97) (width 0.2) (layer "B.Cu") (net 12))
 (segment (start 146.5087 90.8287) (end 145.3 89.62) (width 0.3) (layer "B.Cu") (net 10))
 (segment (start 167.6463 90.8287) (end 146.5087 90.8287) (width 0.3) (layer "B.Cu") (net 10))
 (segment (start 168.075 90.4) (end 167.6463 90.8287) (width 0.3) (layer "B.Cu") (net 10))
 (segment (start 168.075 93.9) (end 167.605 93.43) (width 0.2) (layer "B.Cu") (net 11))
 (segment (start 146.57 93.43) (end 145.3 92.16) (width 0.2) (layer "B.Cu") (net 11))
 (segment (start 167.605 93.43) (end 146.57 93.43) (width 0.2) (layer "B.Cu") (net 11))
 (segment (start 149.16 104.56) (end 150.5917 104.56) (width 0.3) (layer "F.Cu") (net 2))
 (segment (start 150.5917 104.56) (end 157.9117 97.24) (width 0.3) (layer "F.Cu") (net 2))
 (segment (start 157.9117 97.24) (end 158 97.24) (width 0.3) (layer "F.Cu") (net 2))
 (segment (start 156.8698 94.7) (end 147.7283 103.8415) (width 0.3) (layer "F.Cu") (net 3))
 (segment (start 158 94.7) (end 156.8698 94.7) (width 0.3) (layer "F.Cu") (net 3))
 (segment (start 147.7283 103.8415) (end 147.7283 107.1) (width 0.3) (layer "F.Cu") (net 3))
 (segment (start 149.16 107.1) (end 147.7283 107.1) (width 0.3) (layer "F.Cu") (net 3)))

